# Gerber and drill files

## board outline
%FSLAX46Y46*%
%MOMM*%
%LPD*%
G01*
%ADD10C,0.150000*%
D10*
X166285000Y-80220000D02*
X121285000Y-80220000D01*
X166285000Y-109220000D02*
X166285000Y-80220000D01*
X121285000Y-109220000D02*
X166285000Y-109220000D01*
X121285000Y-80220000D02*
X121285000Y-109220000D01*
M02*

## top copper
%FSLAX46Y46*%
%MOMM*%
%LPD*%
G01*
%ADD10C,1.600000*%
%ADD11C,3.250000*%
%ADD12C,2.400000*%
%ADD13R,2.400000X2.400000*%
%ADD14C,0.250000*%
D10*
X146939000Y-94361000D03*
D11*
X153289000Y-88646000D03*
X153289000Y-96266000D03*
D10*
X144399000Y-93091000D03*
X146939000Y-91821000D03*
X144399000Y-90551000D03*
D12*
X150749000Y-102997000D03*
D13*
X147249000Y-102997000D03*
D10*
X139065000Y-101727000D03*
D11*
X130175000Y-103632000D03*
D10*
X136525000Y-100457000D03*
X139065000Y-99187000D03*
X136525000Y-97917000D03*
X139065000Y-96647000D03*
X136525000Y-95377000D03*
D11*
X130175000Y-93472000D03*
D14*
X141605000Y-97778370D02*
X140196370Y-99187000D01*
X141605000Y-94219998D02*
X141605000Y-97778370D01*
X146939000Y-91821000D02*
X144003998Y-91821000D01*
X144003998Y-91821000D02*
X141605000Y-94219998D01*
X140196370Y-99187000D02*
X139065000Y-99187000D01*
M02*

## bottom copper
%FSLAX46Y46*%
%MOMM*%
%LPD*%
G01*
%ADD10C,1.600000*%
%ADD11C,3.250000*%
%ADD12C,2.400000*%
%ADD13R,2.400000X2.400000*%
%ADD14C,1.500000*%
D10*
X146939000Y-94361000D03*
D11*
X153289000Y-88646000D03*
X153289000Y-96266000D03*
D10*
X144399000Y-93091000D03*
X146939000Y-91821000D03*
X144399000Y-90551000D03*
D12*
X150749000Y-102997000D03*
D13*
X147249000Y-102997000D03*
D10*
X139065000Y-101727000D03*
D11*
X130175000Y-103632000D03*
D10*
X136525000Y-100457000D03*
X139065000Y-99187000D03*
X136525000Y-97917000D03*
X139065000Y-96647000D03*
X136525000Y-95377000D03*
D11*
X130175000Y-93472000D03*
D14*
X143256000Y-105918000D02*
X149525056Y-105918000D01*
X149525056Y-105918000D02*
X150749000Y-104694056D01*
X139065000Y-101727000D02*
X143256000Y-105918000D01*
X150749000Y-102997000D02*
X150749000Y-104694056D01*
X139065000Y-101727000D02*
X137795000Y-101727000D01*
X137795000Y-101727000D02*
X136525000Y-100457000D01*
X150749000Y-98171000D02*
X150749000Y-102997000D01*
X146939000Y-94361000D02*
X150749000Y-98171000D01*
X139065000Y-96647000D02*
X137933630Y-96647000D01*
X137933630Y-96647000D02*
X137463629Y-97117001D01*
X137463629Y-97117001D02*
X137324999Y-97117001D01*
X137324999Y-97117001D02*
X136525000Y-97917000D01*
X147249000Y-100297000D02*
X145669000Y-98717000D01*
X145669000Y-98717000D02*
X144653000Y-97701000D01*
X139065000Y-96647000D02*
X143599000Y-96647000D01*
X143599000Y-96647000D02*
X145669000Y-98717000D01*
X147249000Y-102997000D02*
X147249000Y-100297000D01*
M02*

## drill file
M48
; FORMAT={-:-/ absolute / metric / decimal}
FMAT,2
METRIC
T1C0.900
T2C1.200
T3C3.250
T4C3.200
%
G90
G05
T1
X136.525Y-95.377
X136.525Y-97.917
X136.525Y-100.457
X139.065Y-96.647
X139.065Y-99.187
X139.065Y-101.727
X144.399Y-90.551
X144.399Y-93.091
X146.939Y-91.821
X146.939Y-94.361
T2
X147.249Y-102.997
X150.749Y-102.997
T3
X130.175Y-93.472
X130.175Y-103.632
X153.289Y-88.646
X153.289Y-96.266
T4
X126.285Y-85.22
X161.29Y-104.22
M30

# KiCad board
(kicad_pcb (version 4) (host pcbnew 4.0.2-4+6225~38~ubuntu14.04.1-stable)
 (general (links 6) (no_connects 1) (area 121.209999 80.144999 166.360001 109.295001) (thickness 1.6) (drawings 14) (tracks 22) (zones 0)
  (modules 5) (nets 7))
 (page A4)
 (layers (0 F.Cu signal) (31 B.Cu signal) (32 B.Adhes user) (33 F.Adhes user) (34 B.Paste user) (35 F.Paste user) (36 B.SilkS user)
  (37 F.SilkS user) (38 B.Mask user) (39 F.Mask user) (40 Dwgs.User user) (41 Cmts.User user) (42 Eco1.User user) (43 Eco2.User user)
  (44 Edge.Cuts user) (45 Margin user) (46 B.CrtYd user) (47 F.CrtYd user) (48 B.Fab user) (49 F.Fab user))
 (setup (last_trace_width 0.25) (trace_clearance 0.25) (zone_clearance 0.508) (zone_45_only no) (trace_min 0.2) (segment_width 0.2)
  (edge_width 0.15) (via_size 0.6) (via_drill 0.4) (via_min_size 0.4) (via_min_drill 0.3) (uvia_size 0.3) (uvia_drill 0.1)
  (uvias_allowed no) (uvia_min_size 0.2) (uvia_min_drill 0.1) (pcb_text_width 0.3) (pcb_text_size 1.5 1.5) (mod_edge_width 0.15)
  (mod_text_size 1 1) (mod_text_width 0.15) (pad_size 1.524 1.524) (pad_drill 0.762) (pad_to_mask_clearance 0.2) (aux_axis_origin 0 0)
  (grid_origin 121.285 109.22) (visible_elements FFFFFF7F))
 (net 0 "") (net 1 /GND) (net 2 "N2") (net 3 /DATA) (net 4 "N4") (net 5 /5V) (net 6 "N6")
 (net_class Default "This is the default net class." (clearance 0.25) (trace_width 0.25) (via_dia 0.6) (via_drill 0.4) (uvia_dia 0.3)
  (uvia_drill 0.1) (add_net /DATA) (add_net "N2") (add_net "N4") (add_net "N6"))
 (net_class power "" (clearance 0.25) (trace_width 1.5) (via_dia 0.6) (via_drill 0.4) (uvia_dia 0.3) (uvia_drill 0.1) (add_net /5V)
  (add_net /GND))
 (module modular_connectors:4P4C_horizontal (layer F.Cu) (at 146.939 94.361 90) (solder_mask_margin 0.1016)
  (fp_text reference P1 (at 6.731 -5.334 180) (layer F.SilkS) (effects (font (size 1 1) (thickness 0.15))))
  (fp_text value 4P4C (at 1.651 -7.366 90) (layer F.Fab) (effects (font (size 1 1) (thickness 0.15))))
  (pad 1 thru_hole circle (at 0 0 90) (size 1.6 1.6) (drill 0.9) (layers *.Cu *.Mask F.SilkS) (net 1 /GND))
  (pad 6 thru_hole circle (at 5.715 6.35 90) (size 3.25 3.25) (drill 3.25) (layers *.Cu *.Mask F.SilkS))
  (pad 5 thru_hole circle (at -1.905 6.35 90) (size 3.25 3.25) (drill 3.25) (layers *.Cu *.Mask F.SilkS))
  (pad 2 thru_hole circle (at 1.27 -2.54 90) (size 1.6 1.6) (drill 0.9) (layers *.Cu *.Mask F.SilkS) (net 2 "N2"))
  (pad 3 thru_hole circle (at 2.54 0 90) (size 1.6 1.6) (drill 0.9) (layers *.Cu *.Mask F.SilkS) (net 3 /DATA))
  (pad 4 thru_hole circle (at 3.81 -2.54 90) (size 1.6 1.6) (drill 0.9) (layers *.Cu *.Mask F.SilkS) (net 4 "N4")))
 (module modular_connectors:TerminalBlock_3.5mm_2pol (layer F.Cu) (at 147.249 102.997)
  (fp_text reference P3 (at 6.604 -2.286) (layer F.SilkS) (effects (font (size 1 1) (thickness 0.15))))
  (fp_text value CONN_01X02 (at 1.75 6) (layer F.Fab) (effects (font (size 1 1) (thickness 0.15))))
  (pad 2 thru_hole circle (at 3.5 0) (size 2.4 2.4) (drill 1.2) (layers *.Cu *.Mask F.SilkS) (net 1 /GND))
  (pad 1 thru_hole rect (at 0 0) (size 2.4 2.4) (drill 1.2) (layers *.Cu *.Mask F.SilkS) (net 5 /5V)))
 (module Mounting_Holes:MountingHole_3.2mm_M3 (layer F.Cu) (at 161.29 104.22)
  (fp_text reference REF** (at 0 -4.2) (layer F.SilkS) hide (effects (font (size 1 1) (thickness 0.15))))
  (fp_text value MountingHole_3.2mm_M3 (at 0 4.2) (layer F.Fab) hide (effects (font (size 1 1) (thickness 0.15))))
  (pad 1 np_thru_hole circle (at 0 0) (size 3.2 3.2) (drill 3.2) (layers *.Cu *.Mask F.SilkS)))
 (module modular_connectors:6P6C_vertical (layer B.Cu) (at 139.065 99.187 90)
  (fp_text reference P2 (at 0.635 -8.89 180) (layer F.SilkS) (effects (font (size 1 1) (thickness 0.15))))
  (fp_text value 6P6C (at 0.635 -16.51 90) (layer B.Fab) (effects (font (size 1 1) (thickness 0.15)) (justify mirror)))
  (pad 1 thru_hole circle (at -2.54 0 90) (size 1.6 1.6) (drill 0.9) (layers *.Cu *.Mask B.SilkS) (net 1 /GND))
  (pad 7 thru_hole circle (at -4.445 -8.89 90) (size 3.25 3.25) (drill 3.25) (layers *.Cu *.Mask B.SilkS))
  (pad 2 thru_hole circle (at -1.27 -2.54 90) (size 1.6 1.6) (drill 0.9) (layers *.Cu *.Mask B.SilkS) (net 1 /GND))
  (pad 3 thru_hole circle (at 0 0 90) (size 1.6 1.6) (drill 0.9) (layers *.Cu *.Mask B.SilkS) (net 3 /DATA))
  (pad 4 thru_hole circle (at 1.27 -2.54 90) (size 1.6 1.6) (drill 0.9) (layers *.Cu *.Mask B.SilkS) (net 5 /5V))
  (pad 5 thru_hole circle (at 2.54 0 90) (size 1.6 1.6) (drill 0.9) (layers *.Cu *.Mask B.SilkS) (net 5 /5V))
  (pad 6 thru_hole circle (at 3.81 -2.54 90) (size 1.6 1.6) (drill 0.9) (layers *.Cu *.Mask B.SilkS) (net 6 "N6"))
  (pad 8 thru_hole circle (at 5.715 -8.89 90) (size 3.25 3.25) (drill 3.25) (layers *.Cu *.Mask B.SilkS)))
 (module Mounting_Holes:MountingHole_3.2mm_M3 (layer F.Cu) (at 126.285 85.22)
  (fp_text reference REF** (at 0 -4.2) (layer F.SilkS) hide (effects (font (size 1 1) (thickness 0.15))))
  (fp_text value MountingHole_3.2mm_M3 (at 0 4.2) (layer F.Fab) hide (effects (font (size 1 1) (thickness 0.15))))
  (pad 1 np_thru_hole circle (at 0 0) (size 3.2 3.2) (drill 3.2) (layers *.Cu *.Mask F.SilkS)))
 (gr_line (start 166.285 80.22) (end 121.285 80.22) (layer Edge.Cuts) (width 0.15))
 (gr_line (start 166.285 109.22) (end 166.285 80.22) (layer Edge.Cuts) (width 0.15))
 (gr_line (start 121.285 109.22) (end 166.285 109.22) (layer Edge.Cuts) (width 0.15))
 (gr_line (start 121.285 80.22) (end 121.285 109.22) (layer Edge.Cuts) (width 0.15))
 (segment (start 143.256 105.918) (end 149.525056 105.918) (width 1.5) (layer B.Cu) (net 1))
 (segment (start 149.525056 105.918) (end 150.749 104.694056) (width 1.5) (layer B.Cu) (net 1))
 (segment (start 139.065 101.727) (end 143.256 105.918) (width 1.5) (layer B.Cu) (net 1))
 (segment (start 150.749 102.997) (end 150.749 104.694056) (width 1.5) (layer B.Cu) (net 1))
 (segment (start 139.065 101.727) (end 137.795 101.727) (width 1.5) (layer B.Cu) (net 1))
 (segment (start 137.795 101.727) (end 136.525 100.457) (width 1.5) (layer B.Cu) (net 1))
 (segment (start 150.749 98.171) (end 150.749 102.997) (width 1.5) (layer B.Cu) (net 1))
 (segment (start 146.939 94.361) (end 150.749 98.171) (width 1.5) (layer B.Cu) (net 1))
 (segment (start 141.605 97.77837) (end 140.19637 99.187) (width 0.25) (layer F.Cu) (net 3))
 (segment (start 141.605 94.219998) (end 141.605 97.77837) (width 0.25) (layer F.Cu) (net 3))
 (segment (start 146.939 91.821) (end 144.003998 91.821) (width 0.25) (layer F.Cu) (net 3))
 (segment (start 144.003998 91.821) (end 141.605 94.219998) (width 0.25) (layer F.Cu) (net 3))
 (segment (start 140.19637 99.187) (end 139.065 99.187) (width 0.25) (layer F.Cu) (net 3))
 (segment (start 139.065 96.647) (end 137.93363 96.647) (width 1.5) (layer B.Cu) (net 5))
 (segment (start 137.93363 96.647) (end 137.463629 97.117001) (width 1.5) (layer B.Cu) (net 5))
 (segment (start 137.463629 97.117001) (end 137.324999 97.117001) (width 1.5) (layer B.Cu) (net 5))
 (segment (start 137.324999 97.117001) (end 136.525 97.917) (width 1.5) (layer B.Cu) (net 5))
 (segment (start 147.249 100.297) (end 145.669 98.717) (width 1.5) (layer B.Cu) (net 5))
 (segment (start 145.669 98.717) (end 144.653 97.701) (width 1.5) (layer B.Cu) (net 5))
 (segment (start 139.065 96.647) (end 143.599 96.647) (width 1.5) (layer B.Cu) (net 5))
 (segment (start 143.599 96.647) (end 145.669 98.717) (width 1.5) (layer B.Cu) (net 5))
 (segment (start 147.249 102.997) (end 147.249 100.297) (width 1.5) (layer B.Cu) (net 5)))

